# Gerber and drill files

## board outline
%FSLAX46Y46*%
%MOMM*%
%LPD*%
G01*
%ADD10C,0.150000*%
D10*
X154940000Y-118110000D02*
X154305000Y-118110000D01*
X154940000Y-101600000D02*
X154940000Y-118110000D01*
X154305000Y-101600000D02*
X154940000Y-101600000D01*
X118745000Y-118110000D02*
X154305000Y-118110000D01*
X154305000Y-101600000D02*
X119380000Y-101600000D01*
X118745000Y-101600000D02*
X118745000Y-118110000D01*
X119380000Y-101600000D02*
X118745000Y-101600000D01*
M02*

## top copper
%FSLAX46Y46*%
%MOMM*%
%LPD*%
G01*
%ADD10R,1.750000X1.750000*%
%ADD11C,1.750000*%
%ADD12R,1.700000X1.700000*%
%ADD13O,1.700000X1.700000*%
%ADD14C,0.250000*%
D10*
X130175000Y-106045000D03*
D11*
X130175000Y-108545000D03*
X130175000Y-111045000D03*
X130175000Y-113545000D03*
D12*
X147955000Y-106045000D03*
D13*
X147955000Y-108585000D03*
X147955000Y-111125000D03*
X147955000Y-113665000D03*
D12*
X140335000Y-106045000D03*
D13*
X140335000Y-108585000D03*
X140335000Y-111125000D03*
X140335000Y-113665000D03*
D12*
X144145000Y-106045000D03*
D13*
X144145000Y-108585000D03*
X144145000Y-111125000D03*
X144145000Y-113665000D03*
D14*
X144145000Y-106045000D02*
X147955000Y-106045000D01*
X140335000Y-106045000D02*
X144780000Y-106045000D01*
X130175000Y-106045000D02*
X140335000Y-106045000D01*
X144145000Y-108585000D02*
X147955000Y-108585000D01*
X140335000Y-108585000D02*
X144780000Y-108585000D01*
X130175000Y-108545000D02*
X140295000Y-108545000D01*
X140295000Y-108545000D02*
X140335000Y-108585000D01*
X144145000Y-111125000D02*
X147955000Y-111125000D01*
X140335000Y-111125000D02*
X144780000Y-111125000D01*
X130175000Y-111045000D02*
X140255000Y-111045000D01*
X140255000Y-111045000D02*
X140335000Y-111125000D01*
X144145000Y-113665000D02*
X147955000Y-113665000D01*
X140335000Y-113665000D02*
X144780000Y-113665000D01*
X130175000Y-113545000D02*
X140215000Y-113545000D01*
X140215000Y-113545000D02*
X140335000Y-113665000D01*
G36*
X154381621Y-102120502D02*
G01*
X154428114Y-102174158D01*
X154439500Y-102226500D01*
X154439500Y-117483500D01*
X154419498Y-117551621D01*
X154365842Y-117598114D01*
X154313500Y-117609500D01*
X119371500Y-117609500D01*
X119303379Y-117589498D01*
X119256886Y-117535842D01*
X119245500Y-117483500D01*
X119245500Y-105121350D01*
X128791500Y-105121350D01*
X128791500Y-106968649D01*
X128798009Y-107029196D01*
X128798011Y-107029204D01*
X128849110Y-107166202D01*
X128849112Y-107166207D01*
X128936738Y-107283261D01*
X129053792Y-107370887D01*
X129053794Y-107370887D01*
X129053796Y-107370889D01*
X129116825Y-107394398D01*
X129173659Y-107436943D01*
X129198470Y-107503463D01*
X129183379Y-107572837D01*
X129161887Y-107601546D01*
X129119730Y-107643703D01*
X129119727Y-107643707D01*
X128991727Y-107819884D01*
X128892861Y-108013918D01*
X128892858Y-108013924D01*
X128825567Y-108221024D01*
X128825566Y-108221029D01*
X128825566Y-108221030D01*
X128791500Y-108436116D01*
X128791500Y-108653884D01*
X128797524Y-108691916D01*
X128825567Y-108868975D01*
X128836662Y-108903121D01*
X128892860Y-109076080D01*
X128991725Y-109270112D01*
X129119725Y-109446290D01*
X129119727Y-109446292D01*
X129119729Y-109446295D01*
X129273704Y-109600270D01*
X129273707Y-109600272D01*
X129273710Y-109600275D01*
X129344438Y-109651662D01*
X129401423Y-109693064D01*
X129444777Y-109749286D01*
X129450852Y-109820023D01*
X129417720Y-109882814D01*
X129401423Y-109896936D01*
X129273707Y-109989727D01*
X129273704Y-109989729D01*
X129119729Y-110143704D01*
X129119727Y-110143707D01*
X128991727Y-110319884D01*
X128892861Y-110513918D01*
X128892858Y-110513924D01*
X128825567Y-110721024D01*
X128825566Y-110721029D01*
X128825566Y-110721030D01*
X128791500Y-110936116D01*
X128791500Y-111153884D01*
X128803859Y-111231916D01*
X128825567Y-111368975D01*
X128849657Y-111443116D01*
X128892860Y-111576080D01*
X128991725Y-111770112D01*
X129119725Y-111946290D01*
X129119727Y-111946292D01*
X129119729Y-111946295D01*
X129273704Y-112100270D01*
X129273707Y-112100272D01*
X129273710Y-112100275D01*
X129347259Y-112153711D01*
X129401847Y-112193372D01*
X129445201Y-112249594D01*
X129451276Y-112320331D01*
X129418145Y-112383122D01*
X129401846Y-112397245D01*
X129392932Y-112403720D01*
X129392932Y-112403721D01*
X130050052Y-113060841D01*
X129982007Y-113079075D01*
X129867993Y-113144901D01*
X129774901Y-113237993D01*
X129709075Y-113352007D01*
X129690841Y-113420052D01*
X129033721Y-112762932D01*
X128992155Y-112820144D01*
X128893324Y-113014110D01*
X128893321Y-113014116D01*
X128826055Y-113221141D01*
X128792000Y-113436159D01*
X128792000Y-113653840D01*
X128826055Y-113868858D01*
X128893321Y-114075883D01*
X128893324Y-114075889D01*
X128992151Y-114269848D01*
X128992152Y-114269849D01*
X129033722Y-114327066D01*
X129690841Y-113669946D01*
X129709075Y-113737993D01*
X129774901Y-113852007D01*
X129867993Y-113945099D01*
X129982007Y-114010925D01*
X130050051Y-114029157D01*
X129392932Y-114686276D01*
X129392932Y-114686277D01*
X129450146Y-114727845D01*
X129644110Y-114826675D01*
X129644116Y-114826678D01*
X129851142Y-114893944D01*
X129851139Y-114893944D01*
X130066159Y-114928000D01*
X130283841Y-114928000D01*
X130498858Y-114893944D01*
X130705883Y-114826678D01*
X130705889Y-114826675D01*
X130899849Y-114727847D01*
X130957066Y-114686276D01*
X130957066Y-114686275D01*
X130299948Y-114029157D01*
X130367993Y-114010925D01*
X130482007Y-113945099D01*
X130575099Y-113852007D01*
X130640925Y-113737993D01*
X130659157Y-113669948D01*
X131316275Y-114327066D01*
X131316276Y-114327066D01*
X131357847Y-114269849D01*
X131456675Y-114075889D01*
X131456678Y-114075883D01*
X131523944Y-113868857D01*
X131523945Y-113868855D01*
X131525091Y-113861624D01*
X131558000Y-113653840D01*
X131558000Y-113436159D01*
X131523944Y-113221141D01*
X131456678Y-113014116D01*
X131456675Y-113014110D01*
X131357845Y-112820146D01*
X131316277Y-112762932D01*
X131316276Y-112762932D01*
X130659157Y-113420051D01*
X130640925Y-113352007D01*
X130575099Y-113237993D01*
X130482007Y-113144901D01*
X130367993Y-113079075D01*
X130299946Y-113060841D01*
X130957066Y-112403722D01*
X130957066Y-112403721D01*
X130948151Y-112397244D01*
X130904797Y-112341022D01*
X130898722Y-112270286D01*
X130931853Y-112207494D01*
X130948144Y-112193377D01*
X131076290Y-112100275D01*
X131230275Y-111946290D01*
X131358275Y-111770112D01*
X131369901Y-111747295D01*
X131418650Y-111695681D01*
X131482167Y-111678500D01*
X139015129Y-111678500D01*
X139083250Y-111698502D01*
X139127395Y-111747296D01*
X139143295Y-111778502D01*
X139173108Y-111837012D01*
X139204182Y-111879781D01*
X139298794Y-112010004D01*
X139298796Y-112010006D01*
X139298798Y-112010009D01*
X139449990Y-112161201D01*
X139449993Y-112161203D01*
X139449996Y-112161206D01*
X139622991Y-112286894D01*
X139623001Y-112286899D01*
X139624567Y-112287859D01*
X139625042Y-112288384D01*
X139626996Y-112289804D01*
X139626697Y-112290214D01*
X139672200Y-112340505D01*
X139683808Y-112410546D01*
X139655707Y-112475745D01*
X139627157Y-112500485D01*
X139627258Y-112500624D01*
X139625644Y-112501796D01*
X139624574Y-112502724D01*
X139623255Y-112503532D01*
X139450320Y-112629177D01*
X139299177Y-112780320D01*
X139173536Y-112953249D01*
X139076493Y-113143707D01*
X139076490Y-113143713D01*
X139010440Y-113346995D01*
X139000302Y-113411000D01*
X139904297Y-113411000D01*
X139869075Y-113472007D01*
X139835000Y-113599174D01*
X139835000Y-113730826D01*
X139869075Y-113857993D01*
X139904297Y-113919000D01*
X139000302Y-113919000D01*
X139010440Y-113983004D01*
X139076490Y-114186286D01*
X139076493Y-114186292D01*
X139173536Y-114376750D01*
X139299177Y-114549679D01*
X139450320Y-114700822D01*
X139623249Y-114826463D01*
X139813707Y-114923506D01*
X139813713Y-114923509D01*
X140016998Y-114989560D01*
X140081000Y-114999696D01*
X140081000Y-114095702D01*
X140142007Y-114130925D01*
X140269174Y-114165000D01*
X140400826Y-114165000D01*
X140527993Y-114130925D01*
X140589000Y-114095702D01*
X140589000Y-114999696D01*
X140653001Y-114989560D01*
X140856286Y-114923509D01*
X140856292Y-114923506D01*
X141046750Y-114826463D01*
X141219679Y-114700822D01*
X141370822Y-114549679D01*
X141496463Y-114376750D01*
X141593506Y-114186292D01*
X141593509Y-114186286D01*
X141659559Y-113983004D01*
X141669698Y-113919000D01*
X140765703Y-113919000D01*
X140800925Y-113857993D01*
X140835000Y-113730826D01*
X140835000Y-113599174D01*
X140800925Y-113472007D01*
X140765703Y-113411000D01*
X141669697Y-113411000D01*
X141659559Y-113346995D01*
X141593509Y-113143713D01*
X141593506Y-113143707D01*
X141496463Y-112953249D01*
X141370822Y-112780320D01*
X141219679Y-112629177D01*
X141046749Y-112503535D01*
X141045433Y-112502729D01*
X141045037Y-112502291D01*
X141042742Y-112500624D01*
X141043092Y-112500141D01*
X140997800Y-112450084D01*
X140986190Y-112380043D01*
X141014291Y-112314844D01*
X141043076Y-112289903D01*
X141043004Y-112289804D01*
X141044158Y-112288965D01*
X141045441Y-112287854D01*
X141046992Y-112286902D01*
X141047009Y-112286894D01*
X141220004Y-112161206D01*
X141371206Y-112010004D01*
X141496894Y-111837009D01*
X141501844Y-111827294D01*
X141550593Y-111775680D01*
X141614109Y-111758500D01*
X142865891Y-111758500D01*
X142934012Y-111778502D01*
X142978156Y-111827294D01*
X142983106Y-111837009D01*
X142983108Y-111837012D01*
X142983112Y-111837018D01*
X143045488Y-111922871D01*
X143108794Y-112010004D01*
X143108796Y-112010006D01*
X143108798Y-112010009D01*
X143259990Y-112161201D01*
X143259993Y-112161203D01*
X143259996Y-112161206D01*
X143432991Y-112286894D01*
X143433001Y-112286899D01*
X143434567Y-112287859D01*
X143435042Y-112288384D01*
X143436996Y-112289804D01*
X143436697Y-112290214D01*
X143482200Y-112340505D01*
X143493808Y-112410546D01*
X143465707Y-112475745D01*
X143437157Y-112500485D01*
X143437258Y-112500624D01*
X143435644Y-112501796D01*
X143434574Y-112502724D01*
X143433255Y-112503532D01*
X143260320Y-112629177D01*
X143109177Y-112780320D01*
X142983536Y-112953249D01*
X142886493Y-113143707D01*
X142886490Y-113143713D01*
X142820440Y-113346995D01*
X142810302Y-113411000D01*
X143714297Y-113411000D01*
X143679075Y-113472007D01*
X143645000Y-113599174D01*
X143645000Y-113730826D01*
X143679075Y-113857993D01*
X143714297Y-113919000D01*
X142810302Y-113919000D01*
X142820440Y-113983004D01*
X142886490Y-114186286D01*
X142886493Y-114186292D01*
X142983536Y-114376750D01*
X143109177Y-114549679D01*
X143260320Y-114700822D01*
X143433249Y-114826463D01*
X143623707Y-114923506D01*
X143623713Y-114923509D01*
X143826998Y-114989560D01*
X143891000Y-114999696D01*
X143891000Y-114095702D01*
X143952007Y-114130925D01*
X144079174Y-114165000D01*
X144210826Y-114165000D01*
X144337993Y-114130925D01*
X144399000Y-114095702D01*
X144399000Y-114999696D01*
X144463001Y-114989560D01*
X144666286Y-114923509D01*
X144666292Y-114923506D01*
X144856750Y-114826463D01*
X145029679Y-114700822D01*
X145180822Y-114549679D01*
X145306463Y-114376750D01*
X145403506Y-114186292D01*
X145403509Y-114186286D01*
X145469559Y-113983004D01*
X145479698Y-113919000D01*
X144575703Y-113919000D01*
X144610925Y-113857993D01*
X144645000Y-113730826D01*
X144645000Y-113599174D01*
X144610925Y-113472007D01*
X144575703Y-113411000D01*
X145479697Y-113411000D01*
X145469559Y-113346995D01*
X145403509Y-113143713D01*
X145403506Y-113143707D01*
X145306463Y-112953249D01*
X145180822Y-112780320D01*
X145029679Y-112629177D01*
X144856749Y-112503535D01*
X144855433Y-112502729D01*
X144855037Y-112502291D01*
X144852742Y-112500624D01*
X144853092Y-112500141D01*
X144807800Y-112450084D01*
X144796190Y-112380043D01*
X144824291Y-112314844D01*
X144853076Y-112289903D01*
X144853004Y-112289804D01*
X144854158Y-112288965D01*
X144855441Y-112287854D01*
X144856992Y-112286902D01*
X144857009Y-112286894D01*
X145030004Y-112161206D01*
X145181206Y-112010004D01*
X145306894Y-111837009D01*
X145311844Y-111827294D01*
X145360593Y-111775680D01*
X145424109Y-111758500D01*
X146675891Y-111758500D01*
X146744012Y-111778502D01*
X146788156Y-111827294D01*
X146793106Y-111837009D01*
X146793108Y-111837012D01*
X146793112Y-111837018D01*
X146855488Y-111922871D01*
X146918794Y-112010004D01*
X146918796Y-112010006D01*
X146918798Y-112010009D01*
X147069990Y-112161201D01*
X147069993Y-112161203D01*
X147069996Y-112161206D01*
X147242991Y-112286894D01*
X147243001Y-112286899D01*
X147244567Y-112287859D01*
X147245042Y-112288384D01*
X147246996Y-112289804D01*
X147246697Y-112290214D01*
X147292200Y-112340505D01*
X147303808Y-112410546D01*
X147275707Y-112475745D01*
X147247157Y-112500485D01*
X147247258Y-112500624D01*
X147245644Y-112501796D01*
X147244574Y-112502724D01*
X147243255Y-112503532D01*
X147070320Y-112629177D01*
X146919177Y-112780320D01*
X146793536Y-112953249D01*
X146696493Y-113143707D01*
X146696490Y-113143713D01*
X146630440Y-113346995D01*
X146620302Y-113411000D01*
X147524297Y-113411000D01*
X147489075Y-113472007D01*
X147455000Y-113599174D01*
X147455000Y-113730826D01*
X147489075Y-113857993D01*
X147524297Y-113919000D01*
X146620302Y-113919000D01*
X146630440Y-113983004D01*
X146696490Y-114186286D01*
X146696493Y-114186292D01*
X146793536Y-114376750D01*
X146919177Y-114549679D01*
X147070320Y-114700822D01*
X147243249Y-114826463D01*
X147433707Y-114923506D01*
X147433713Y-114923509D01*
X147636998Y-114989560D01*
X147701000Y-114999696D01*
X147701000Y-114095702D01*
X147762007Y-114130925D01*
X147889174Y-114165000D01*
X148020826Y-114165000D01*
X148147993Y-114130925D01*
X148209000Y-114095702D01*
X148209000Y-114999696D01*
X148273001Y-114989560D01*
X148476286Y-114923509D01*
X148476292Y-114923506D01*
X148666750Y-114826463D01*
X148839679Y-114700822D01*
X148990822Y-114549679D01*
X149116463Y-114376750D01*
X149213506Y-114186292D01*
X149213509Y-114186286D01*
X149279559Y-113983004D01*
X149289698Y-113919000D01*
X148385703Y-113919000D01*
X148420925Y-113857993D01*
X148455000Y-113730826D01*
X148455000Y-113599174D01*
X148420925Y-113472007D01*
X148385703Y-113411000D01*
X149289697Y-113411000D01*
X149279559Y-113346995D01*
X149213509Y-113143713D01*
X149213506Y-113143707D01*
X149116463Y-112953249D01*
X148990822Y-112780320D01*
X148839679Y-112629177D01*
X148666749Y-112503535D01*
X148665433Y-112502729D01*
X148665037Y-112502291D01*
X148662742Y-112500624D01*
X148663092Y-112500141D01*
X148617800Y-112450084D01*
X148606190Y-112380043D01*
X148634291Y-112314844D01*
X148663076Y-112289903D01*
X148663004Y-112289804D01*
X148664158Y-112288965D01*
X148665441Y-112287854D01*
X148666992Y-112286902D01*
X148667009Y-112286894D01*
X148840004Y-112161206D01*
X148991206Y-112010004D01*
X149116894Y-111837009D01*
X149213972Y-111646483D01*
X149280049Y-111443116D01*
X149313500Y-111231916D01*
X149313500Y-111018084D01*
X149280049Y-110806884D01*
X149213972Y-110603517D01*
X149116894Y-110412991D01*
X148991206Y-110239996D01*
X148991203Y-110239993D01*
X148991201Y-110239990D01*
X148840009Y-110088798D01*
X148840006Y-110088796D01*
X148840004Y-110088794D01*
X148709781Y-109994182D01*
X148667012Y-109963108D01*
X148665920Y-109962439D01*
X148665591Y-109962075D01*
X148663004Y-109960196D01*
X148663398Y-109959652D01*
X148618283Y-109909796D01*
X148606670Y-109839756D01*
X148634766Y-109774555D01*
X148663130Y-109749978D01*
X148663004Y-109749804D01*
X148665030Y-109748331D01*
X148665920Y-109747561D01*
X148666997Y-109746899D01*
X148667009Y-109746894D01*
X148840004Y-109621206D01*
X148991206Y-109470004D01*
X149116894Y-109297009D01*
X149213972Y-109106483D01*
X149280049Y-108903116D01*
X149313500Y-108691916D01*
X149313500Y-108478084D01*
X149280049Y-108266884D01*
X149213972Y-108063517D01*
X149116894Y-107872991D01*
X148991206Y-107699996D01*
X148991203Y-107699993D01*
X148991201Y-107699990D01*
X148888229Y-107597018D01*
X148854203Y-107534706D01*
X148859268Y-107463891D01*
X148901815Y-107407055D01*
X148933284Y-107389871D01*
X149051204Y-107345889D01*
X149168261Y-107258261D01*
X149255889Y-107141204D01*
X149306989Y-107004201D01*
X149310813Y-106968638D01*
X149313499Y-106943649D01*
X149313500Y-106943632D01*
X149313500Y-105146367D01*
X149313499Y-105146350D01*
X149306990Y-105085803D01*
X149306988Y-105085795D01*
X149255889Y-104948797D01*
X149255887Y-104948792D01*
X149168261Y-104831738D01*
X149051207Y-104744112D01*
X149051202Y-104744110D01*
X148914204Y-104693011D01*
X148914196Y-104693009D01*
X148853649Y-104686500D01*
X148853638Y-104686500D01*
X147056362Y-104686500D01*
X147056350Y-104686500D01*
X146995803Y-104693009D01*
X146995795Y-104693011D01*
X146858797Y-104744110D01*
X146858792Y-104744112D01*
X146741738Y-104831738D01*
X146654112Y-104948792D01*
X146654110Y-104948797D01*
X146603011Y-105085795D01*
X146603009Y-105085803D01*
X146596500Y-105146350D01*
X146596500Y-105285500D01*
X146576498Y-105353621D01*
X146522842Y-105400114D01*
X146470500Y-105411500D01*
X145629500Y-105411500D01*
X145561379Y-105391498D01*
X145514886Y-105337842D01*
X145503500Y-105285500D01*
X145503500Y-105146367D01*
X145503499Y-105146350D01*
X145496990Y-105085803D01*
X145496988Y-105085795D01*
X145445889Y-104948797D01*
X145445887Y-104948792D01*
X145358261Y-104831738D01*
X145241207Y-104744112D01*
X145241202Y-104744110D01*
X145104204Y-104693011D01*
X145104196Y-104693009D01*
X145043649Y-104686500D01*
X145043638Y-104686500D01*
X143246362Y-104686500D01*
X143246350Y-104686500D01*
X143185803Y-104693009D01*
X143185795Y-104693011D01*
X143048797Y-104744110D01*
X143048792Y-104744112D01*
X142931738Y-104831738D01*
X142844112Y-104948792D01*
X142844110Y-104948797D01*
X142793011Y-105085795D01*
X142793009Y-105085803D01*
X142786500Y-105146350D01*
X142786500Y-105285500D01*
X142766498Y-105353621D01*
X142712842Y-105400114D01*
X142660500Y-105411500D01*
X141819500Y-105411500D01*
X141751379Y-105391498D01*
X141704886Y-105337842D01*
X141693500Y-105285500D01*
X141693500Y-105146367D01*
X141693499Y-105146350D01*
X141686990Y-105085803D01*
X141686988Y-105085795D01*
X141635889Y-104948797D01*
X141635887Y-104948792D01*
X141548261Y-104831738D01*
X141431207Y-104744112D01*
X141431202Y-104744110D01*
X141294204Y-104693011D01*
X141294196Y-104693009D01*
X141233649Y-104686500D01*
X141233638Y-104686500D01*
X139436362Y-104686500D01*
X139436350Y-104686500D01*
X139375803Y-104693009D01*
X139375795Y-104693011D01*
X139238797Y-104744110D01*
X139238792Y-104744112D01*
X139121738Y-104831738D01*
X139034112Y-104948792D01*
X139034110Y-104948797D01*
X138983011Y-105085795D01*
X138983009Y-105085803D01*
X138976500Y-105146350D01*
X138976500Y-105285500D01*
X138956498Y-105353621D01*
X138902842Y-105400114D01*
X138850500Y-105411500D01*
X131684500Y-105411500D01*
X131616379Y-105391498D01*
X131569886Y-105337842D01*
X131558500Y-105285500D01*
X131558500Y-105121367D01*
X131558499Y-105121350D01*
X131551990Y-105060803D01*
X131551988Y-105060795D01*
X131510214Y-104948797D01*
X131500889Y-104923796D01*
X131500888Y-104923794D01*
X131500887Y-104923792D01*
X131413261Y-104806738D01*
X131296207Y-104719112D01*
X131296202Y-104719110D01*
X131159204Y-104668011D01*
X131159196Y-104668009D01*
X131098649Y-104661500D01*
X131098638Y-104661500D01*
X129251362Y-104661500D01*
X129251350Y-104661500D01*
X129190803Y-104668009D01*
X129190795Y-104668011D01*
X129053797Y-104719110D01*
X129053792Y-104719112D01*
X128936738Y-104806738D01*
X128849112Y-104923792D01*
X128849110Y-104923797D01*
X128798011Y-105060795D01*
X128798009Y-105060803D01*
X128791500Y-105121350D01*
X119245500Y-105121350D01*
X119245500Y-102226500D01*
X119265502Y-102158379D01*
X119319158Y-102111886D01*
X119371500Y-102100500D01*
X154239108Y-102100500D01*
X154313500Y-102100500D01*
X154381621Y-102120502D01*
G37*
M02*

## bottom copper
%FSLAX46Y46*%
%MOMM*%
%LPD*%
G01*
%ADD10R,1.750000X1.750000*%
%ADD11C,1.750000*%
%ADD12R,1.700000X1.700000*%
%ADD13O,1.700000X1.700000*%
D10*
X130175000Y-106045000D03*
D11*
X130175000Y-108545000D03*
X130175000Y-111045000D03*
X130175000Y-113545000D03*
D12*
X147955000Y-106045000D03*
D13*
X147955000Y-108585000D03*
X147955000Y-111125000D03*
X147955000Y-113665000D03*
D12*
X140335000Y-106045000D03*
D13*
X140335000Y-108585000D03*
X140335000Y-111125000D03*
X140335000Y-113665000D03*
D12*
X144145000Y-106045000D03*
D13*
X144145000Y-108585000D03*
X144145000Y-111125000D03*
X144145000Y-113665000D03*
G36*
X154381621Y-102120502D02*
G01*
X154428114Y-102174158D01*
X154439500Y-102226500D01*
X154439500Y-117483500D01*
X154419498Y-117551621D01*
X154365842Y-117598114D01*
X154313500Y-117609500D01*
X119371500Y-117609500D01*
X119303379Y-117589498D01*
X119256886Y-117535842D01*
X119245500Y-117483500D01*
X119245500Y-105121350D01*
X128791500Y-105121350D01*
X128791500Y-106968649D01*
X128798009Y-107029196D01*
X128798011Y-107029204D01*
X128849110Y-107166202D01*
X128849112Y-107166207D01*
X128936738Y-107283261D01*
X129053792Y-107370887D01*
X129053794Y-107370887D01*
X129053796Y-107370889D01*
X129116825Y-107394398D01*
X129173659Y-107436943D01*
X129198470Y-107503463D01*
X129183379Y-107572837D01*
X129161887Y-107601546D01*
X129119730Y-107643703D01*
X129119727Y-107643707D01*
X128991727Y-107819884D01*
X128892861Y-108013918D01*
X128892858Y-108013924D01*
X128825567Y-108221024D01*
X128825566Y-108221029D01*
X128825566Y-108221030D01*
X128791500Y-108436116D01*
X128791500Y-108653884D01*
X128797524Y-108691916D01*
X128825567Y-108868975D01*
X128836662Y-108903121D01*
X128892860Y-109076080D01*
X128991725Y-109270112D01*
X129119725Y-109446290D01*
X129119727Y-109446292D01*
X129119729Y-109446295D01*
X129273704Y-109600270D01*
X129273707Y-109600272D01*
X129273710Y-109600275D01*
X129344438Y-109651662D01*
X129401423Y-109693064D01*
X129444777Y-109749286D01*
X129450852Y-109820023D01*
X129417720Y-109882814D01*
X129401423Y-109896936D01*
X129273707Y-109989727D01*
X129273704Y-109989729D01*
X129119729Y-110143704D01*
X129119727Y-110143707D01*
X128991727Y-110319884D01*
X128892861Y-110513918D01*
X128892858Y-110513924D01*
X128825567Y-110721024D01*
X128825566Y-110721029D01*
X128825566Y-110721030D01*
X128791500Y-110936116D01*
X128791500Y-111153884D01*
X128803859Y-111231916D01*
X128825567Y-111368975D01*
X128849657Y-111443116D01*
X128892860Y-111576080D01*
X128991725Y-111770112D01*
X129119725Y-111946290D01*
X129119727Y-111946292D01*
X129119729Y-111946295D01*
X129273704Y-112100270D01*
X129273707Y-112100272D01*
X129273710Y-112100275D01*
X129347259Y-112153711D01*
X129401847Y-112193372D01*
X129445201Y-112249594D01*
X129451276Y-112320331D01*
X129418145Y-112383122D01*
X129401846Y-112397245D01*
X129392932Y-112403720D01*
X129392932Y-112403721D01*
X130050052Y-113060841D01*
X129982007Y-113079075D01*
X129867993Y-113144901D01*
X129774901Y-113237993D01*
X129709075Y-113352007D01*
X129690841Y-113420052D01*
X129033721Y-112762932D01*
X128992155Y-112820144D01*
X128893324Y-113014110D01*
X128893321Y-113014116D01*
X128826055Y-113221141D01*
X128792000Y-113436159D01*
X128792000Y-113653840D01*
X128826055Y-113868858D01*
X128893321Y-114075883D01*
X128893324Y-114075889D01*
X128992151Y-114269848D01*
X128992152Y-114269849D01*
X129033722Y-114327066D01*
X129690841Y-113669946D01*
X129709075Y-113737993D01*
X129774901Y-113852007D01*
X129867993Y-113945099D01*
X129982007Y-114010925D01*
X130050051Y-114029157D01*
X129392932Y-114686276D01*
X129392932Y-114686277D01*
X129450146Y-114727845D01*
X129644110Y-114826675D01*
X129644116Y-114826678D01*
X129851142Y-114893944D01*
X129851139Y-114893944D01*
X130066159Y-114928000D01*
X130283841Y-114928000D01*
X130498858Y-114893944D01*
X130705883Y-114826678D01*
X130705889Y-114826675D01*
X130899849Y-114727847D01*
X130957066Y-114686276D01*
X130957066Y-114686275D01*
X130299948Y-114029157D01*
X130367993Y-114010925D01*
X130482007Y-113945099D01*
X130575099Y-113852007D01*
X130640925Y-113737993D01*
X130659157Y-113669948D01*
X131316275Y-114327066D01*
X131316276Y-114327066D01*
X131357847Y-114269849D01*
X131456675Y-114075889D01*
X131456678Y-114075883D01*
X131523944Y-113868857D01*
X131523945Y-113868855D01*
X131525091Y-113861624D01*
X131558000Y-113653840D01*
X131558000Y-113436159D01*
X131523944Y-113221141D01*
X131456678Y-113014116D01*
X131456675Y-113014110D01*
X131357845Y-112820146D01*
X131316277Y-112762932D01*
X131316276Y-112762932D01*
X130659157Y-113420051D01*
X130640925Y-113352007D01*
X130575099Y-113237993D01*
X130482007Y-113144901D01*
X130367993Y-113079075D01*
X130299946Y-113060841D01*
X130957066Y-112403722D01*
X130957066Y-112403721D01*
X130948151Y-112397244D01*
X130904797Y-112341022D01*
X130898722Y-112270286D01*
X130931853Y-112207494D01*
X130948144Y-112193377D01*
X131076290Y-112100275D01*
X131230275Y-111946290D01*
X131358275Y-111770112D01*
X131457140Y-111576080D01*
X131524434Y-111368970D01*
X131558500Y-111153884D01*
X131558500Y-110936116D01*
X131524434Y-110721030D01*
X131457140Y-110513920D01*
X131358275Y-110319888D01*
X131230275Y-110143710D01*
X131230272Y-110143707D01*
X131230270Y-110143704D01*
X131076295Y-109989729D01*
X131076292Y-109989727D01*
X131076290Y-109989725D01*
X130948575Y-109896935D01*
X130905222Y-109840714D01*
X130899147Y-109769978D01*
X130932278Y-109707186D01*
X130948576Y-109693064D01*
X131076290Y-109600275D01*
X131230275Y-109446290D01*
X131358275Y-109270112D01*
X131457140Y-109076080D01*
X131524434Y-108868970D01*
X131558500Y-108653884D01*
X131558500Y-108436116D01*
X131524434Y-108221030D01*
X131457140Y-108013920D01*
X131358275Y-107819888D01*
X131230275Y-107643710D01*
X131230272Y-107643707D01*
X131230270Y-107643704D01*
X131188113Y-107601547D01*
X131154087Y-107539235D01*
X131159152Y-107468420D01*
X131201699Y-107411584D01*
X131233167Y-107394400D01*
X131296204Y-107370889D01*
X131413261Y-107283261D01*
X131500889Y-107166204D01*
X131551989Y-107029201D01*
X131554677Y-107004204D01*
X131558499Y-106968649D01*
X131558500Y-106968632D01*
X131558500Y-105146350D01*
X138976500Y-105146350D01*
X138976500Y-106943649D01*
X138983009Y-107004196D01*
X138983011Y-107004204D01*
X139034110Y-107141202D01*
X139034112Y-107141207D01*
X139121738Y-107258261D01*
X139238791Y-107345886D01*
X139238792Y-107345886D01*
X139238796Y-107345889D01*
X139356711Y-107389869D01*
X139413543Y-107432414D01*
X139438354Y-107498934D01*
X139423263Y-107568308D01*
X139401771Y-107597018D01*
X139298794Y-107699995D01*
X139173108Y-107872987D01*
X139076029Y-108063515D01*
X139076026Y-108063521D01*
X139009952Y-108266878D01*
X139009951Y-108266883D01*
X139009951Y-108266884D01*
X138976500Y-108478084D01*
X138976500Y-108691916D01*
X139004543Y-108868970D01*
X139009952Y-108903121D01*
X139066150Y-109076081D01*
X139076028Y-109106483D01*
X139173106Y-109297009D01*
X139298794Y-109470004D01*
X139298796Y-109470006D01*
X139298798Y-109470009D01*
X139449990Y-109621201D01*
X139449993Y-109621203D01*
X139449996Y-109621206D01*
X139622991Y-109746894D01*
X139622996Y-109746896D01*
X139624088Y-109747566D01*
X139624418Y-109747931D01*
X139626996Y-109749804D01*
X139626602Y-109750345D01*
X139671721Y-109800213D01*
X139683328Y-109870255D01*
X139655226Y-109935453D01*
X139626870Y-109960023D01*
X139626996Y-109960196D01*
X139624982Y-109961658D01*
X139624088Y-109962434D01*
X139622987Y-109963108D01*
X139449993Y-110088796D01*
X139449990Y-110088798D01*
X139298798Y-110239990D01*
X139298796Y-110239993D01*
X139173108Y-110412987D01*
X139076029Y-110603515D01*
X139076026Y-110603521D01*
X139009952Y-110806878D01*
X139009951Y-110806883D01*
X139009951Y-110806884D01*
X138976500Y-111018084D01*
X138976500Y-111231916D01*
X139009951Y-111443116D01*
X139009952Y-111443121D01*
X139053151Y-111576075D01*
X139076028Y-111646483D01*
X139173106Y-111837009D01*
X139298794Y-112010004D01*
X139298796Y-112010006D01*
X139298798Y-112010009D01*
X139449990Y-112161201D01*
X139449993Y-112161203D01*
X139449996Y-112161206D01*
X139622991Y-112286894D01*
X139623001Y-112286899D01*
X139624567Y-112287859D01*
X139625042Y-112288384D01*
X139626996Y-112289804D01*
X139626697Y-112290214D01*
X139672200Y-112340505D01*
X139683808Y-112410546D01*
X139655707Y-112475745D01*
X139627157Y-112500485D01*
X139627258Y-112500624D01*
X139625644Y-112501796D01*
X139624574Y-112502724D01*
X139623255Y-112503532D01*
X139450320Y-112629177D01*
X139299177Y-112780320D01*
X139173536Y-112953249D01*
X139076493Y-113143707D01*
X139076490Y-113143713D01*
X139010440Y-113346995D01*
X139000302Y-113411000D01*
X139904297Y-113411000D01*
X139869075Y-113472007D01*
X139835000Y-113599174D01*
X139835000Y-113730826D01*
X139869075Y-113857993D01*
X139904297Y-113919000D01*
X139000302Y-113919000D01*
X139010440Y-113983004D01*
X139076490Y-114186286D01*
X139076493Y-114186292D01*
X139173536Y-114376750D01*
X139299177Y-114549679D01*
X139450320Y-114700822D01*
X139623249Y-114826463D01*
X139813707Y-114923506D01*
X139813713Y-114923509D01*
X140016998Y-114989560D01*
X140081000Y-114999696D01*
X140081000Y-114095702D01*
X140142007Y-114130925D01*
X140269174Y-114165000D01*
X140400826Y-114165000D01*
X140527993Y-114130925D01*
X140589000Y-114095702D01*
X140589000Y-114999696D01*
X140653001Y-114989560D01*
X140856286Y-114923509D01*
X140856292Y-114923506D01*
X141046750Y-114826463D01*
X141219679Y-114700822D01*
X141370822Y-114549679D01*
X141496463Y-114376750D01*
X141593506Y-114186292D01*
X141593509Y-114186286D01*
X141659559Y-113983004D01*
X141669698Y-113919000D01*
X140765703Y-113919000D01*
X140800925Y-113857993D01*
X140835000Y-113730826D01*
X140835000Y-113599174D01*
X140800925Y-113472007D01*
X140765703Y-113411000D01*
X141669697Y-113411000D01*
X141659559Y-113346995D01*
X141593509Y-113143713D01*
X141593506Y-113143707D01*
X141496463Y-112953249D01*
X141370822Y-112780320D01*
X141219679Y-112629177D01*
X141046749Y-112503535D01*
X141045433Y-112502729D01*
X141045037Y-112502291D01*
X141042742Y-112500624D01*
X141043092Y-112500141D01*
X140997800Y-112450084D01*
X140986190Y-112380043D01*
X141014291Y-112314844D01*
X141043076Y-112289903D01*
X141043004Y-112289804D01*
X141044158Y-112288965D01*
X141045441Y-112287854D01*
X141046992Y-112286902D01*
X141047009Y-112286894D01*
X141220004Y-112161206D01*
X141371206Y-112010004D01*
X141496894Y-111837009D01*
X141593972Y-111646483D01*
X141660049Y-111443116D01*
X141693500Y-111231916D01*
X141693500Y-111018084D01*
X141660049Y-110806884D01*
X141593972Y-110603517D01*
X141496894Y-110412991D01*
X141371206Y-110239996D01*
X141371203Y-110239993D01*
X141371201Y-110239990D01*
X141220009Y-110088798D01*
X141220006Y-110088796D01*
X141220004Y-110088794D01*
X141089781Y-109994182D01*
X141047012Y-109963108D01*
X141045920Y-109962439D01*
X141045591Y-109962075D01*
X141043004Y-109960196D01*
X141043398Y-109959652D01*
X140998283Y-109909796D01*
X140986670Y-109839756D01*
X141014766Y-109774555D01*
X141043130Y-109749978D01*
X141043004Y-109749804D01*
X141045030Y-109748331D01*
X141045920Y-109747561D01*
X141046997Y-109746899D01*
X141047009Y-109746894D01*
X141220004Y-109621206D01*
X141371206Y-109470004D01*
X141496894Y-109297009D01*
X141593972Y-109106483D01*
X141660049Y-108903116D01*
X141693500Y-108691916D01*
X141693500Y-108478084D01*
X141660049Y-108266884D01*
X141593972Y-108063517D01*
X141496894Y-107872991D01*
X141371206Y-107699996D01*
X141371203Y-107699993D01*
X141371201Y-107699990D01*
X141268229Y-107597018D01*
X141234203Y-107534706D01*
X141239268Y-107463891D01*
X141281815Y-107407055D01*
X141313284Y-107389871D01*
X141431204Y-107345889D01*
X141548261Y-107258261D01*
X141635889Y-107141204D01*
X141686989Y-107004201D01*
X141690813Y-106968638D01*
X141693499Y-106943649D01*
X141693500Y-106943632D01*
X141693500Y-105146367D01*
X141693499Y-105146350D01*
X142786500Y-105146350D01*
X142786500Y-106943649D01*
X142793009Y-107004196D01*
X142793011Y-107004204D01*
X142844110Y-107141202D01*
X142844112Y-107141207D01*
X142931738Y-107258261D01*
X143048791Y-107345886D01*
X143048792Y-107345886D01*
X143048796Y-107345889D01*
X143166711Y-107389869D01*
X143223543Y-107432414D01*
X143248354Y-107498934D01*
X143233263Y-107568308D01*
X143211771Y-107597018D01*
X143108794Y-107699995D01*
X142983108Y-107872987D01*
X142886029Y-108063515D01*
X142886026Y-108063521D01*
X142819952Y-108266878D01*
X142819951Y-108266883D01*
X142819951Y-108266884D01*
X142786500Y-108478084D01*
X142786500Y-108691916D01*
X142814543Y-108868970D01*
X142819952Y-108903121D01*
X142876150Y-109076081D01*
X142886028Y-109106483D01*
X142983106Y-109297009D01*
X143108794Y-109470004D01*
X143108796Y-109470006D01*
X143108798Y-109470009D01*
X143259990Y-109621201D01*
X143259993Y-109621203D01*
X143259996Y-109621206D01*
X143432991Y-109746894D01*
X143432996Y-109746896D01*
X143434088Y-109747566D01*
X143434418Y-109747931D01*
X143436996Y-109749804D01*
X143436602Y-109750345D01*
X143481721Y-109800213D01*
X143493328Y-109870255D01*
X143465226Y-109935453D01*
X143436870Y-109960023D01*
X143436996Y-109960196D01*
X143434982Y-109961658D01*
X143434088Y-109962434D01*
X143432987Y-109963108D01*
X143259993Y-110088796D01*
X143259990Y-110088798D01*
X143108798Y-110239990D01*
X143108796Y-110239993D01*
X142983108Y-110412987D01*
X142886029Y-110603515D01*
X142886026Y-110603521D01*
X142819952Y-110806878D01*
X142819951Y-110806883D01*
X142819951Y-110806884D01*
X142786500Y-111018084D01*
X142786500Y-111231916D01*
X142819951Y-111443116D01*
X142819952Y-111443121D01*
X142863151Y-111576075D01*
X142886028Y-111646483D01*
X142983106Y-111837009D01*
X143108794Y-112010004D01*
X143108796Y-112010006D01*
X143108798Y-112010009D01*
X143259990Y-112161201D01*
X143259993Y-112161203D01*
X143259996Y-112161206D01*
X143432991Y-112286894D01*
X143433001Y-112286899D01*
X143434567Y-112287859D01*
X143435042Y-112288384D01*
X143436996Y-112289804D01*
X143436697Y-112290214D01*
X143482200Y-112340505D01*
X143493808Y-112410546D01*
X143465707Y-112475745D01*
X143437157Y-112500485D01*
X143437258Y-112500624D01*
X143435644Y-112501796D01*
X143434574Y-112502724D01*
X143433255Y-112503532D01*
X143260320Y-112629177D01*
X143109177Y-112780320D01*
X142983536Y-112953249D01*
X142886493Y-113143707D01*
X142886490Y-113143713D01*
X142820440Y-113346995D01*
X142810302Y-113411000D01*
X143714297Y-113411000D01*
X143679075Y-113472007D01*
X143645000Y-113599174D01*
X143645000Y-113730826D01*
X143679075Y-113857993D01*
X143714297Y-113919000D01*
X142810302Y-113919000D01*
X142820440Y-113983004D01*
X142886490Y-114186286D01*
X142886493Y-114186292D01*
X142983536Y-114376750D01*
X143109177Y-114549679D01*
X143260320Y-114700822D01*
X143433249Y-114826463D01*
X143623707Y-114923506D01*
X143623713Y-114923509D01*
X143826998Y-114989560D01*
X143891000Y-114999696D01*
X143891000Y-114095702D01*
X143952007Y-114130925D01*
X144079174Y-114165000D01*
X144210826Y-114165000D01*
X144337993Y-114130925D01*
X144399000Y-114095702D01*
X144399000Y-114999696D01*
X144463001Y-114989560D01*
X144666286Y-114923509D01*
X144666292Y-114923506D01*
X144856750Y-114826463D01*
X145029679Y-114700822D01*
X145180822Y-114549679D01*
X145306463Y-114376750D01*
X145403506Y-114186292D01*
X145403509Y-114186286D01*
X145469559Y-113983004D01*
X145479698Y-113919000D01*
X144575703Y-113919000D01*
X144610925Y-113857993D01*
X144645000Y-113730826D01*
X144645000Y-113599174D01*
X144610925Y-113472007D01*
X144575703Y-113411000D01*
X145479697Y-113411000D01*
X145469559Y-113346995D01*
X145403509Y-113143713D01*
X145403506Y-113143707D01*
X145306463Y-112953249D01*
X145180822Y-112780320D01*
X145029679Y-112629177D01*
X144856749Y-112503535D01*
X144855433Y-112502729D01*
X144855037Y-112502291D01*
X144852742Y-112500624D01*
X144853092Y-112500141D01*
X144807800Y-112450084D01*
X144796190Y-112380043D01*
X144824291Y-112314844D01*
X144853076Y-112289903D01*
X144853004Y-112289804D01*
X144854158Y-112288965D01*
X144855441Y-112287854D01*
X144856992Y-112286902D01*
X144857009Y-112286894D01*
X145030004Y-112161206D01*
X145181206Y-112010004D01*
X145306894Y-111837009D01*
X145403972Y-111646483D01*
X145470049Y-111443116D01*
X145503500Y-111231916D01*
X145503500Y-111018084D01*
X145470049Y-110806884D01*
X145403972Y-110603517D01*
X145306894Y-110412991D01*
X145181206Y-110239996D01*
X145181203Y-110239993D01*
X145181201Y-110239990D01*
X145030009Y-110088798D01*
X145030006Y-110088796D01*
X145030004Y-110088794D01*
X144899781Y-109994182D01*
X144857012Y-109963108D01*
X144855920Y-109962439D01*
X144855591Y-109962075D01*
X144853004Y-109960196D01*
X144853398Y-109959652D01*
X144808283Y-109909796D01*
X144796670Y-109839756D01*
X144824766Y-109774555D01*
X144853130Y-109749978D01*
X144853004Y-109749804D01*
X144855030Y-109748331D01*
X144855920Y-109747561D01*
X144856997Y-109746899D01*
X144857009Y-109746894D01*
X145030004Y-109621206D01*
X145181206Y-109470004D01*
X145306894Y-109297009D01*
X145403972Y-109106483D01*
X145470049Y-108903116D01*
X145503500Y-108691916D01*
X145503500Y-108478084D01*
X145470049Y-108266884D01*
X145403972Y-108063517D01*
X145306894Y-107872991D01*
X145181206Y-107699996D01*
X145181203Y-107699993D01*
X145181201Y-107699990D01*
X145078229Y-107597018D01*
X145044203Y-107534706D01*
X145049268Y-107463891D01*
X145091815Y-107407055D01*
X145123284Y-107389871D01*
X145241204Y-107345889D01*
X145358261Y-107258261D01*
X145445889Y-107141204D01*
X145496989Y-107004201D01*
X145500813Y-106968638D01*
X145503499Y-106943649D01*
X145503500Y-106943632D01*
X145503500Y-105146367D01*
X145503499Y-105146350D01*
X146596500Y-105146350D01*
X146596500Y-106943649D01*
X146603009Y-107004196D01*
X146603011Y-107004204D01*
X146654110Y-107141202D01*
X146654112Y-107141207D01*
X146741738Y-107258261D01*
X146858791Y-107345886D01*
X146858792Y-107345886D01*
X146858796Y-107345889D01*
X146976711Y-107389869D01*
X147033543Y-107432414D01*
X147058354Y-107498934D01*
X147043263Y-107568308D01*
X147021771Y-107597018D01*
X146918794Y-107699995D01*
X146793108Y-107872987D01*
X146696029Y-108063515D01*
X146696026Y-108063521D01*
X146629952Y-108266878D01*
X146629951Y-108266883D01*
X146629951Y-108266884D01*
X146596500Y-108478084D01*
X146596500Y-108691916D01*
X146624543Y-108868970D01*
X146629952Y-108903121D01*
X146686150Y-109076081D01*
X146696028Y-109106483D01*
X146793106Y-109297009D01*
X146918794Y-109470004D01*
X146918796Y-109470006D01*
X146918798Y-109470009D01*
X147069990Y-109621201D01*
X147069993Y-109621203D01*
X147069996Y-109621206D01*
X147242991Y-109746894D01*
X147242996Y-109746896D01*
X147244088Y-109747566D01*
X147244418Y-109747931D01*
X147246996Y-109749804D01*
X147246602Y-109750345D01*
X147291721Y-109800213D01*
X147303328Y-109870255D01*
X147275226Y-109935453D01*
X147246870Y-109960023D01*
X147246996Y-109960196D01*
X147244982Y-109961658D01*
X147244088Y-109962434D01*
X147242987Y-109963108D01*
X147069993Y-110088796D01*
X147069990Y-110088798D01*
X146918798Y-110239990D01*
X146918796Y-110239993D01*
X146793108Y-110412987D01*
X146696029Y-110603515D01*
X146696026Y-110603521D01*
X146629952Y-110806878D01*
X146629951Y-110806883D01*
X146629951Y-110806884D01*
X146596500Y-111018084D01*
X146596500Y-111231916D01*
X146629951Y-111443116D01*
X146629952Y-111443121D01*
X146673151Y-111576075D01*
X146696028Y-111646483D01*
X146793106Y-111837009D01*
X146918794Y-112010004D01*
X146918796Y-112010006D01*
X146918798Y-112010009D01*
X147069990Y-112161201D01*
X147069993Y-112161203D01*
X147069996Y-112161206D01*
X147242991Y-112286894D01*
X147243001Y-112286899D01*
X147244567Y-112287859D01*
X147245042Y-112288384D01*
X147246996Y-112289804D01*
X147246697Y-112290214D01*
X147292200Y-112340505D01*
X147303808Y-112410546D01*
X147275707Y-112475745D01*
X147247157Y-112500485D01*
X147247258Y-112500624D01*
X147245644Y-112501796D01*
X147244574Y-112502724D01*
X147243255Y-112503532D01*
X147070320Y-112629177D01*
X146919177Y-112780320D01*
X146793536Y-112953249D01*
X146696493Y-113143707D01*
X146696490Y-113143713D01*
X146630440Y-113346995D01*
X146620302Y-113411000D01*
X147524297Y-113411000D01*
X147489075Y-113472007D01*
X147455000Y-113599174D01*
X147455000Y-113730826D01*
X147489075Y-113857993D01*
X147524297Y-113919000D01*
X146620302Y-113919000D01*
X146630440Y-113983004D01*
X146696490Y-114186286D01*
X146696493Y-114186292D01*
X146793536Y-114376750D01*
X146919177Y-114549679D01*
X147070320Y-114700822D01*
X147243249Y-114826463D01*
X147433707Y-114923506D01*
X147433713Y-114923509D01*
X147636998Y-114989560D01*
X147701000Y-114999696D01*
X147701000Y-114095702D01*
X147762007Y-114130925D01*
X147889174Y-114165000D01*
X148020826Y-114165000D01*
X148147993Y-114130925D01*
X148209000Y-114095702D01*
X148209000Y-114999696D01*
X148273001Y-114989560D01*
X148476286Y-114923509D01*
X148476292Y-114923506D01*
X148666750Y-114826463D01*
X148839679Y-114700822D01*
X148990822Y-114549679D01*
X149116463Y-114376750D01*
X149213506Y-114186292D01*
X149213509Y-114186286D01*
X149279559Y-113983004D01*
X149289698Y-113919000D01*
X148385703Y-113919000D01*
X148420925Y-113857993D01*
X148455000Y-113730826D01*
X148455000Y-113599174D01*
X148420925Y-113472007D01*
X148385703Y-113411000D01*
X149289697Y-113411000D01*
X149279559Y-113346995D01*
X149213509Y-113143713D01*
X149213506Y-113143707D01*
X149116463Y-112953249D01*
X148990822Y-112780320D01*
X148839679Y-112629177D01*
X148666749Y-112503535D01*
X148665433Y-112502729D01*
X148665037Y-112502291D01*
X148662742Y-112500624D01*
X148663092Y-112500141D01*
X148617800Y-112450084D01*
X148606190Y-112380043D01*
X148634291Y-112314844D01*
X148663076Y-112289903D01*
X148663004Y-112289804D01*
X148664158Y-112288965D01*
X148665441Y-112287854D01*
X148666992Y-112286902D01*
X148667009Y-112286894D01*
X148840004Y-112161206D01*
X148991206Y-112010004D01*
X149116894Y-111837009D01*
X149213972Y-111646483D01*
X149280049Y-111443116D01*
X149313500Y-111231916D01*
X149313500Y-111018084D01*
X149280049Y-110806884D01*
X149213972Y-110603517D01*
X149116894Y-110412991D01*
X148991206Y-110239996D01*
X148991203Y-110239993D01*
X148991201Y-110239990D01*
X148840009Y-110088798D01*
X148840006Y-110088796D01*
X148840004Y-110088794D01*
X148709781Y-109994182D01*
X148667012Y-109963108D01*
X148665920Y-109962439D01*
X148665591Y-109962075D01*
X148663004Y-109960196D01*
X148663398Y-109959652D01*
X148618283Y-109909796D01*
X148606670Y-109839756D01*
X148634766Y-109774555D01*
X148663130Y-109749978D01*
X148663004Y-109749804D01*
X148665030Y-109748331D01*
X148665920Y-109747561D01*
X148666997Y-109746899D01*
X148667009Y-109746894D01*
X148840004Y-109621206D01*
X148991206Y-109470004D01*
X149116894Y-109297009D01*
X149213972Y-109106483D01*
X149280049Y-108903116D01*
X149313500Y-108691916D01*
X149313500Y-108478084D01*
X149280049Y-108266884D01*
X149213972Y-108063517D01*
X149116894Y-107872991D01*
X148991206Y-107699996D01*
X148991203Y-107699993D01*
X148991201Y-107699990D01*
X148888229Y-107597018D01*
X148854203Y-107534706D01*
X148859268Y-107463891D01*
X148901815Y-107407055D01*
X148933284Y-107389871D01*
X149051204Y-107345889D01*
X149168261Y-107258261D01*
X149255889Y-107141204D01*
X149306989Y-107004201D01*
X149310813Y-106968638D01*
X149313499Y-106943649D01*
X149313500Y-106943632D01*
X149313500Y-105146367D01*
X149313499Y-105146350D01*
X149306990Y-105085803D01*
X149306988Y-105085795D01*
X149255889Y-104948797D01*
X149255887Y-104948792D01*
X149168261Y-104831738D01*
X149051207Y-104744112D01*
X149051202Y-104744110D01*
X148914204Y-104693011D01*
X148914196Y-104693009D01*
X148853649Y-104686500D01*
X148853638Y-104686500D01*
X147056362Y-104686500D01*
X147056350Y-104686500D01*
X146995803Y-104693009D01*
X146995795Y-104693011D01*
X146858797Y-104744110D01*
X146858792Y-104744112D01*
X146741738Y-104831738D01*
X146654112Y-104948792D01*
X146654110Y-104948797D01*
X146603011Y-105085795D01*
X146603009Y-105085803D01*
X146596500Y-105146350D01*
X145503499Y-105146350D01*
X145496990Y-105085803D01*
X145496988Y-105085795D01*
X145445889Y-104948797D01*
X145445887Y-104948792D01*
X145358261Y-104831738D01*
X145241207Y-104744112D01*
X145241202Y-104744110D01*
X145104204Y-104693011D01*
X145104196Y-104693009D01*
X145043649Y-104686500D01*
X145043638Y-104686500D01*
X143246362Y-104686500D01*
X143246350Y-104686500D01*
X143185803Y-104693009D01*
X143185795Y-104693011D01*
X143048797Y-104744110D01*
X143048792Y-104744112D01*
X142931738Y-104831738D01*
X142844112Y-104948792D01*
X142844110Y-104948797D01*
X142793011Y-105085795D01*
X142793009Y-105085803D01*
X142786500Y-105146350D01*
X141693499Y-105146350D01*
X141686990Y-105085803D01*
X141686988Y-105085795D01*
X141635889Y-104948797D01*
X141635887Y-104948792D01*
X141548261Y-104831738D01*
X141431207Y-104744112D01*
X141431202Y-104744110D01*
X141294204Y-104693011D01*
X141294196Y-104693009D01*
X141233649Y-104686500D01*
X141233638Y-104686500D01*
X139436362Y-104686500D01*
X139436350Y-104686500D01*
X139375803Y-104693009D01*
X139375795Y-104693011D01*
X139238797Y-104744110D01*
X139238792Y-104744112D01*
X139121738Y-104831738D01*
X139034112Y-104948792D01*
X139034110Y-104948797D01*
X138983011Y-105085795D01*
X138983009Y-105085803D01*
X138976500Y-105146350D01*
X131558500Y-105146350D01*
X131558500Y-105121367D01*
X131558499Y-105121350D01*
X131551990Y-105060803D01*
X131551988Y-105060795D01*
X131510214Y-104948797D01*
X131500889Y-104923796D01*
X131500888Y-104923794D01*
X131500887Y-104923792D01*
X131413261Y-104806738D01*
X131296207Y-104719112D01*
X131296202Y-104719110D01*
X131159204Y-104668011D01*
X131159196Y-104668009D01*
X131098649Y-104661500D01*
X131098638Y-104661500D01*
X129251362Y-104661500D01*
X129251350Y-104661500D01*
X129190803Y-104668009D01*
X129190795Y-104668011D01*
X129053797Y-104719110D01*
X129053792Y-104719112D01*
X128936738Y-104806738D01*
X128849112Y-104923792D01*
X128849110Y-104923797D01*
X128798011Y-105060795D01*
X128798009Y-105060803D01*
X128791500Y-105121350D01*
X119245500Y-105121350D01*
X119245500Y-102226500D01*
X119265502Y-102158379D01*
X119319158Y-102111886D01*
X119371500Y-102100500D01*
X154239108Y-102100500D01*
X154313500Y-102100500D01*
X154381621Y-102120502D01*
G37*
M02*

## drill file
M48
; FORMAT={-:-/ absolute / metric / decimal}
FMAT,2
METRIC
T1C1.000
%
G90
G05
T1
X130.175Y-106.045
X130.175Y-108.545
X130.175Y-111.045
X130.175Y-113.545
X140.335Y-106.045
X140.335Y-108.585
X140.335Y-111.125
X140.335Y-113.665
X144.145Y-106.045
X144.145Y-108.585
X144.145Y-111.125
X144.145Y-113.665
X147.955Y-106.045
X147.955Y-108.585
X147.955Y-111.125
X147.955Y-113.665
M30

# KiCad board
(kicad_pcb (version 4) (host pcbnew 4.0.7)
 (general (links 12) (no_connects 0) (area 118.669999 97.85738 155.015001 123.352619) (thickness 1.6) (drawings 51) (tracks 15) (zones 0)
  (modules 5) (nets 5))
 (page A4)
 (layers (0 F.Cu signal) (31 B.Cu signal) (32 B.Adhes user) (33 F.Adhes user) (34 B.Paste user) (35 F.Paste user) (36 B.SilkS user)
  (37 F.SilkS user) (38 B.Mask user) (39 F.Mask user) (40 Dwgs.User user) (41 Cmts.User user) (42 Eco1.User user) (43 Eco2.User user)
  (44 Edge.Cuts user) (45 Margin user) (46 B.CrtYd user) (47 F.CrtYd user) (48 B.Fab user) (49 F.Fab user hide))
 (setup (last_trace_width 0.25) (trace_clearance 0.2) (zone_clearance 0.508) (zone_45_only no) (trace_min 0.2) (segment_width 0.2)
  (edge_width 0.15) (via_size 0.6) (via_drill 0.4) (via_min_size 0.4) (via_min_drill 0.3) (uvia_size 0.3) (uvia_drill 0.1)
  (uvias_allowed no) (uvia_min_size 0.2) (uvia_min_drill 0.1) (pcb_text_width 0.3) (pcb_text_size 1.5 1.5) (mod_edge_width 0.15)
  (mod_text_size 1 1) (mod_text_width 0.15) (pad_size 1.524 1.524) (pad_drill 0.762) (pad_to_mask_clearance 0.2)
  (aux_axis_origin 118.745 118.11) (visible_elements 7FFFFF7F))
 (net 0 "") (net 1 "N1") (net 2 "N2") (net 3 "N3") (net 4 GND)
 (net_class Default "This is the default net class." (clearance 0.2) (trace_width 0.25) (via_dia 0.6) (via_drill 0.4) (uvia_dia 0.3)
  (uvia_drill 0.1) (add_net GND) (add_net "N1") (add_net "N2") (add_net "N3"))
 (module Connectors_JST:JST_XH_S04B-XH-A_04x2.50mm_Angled (layer F.Cu) (at 130.175 106.045 270)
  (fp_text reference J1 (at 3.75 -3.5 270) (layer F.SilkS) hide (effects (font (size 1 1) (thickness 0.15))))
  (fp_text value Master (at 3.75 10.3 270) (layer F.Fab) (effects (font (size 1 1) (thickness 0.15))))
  (pad 1 thru_hole rect (at 0 0 270) (size 1.75 1.75) (drill 1) (layers *.Cu *.Mask F.SilkS) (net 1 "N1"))
  (pad 2 thru_hole circle (at 2.5 0 270) (size 1.75 1.75) (drill 1) (layers *.Cu *.Mask F.SilkS) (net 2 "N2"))
  (pad 3 thru_hole circle (at 5 0 270) (size 1.75 1.75) (drill 1) (layers *.Cu *.Mask F.SilkS) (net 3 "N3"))
  (pad 4 thru_hole circle (at 7.5 0 270) (size 1.75 1.75) (drill 1) (layers *.Cu *.Mask F.SilkS) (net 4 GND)))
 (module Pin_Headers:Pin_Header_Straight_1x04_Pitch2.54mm (layer F.Cu) (at 147.955 106.045)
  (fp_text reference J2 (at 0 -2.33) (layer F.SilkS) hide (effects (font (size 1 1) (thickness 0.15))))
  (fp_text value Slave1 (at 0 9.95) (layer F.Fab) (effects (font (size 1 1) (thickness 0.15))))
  (pad 1 thru_hole rect (at 0 0) (size 1.7 1.7) (drill 1) (layers *.Cu *.Mask) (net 1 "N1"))
  (pad 2 thru_hole oval (at 0 2.54) (size 1.7 1.7) (drill 1) (layers *.Cu *.Mask) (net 2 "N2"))
  (pad 3 thru_hole oval (at 0 5.08) (size 1.7 1.7) (drill 1) (layers *.Cu *.Mask) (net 3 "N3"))
  (pad 4 thru_hole oval (at 0 7.62) (size 1.7 1.7) (drill 1) (layers *.Cu *.Mask) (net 4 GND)))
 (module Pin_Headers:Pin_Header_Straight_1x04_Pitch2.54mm (layer F.Cu) (at 140.335 106.045)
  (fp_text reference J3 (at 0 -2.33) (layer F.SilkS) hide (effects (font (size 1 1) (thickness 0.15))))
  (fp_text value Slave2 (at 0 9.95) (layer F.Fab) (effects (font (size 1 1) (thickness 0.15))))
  (pad 1 thru_hole rect (at 0 0) (size 1.7 1.7) (drill 1) (layers *.Cu *.Mask) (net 1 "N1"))
  (pad 2 thru_hole oval (at 0 2.54) (size 1.7 1.7) (drill 1) (layers *.Cu *.Mask) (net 2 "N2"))
  (pad 3 thru_hole oval (at 0 5.08) (size 1.7 1.7) (drill 1) (layers *.Cu *.Mask) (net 3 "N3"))
  (pad 4 thru_hole oval (at 0 7.62) (size 1.7 1.7) (drill 1) (layers *.Cu *.Mask) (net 4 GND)))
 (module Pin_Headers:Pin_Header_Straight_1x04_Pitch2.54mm (layer F.Cu) (at 144.145 106.045)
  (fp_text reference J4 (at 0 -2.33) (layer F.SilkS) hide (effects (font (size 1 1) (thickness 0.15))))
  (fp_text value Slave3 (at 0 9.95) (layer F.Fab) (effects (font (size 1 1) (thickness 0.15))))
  (pad 1 thru_hole rect (at 0 0) (size 1.7 1.7) (drill 1) (layers *.Cu *.Mask) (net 1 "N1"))
  (pad 2 thru_hole oval (at 0 2.54) (size 1.7 1.7) (drill 1) (layers *.Cu *.Mask) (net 2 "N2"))
  (pad 3 thru_hole oval (at 0 5.08) (size 1.7 1.7) (drill 1) (layers *.Cu *.Mask) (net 3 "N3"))
  (pad 4 thru_hole oval (at 0 7.62) (size 1.7 1.7) (drill 1) (layers *.Cu *.Mask) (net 4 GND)))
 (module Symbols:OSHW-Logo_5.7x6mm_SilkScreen (layer B.Cu) (at 135.255 109.855 270)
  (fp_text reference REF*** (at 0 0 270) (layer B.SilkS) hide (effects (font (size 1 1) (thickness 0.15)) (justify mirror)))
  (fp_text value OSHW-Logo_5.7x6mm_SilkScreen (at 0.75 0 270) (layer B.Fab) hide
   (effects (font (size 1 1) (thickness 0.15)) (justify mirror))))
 (gr_line (start 154.94 118.11) (end 154.305 118.11) (layer Edge.Cuts) (width 0.15))
 (gr_line (start 154.94 101.6) (end 154.94 118.11) (layer Edge.Cuts) (width 0.15))
 (gr_line (start 154.305 101.6) (end 154.94 101.6) (layer Edge.Cuts) (width 0.15))
 (gr_line (start 118.745 118.11) (end 154.305 118.11) (layer Edge.Cuts) (width 0.15))
 (gr_line (start 154.305 101.6) (end 119.38 101.6) (layer Edge.Cuts) (width 0.15))
 (gr_line (start 118.745 101.6) (end 118.745 118.11) (layer Edge.Cuts) (width 0.15))
 (gr_line (start 119.38 101.6) (end 118.745 101.6) (layer Edge.Cuts) (width 0.15))
 (segment (start 144.145 106.045) (end 147.955 106.045) (width 0.25) (layer F.Cu) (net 1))
 (segment (start 140.335 106.045) (end 144.78 106.045) (width 0.25) (layer F.Cu) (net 1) (status 30))
 (segment (start 130.175 106.045) (end 140.335 106.045) (width 0.25) (layer F.Cu) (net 1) (status 30))
 (segment (start 144.145 108.585) (end 147.955 108.585) (width 0.25) (layer F.Cu) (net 2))
 (segment (start 140.335 108.585) (end 144.78 108.585) (width 0.25) (layer F.Cu) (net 2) (status 30))
 (segment (start 130.175 108.545) (end 140.295 108.545) (width 0.25) (layer F.Cu) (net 2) (status 30))
 (segment (start 140.295 108.545) (end 140.335 108.585) (width 0.25) (layer F.Cu) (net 2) (status 30))
 (segment (start 144.145 111.125) (end 147.955 111.125) (width 0.25) (layer F.Cu) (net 3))
 (segment (start 140.335 111.125) (end 144.78 111.125) (width 0.25) (layer F.Cu) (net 3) (status 30))
 (segment (start 130.175 111.045) (end 140.255 111.045) (width 0.25) (layer F.Cu) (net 3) (status 30))
 (segment (start 140.255 111.045) (end 140.335 111.125) (width 0.25) (layer F.Cu) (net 3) (status 30))
 (segment (start 144.145 113.665) (end 147.955 113.665) (width 0.25) (layer F.Cu) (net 4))
 (segment (start 140.335 113.665) (end 144.78 113.665) (width 0.25) (layer F.Cu) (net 4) (status 30))
 (segment (start 130.175 113.545) (end 140.215 113.545) (width 0.25) (layer F.Cu) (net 4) (status 30))
 (segment (start 140.215 113.545) (end 140.335 113.665) (width 0.25) (layer F.Cu) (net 4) (status 30))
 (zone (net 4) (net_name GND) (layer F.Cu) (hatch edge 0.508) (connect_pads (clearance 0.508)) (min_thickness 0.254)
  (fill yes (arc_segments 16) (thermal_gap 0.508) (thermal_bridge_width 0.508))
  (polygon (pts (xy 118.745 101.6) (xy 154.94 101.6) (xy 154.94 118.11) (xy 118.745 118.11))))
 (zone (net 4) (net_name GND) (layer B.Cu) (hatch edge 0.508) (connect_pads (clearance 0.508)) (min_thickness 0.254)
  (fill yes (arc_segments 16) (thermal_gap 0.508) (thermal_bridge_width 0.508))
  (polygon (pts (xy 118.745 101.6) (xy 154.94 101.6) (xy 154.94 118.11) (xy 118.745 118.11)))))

